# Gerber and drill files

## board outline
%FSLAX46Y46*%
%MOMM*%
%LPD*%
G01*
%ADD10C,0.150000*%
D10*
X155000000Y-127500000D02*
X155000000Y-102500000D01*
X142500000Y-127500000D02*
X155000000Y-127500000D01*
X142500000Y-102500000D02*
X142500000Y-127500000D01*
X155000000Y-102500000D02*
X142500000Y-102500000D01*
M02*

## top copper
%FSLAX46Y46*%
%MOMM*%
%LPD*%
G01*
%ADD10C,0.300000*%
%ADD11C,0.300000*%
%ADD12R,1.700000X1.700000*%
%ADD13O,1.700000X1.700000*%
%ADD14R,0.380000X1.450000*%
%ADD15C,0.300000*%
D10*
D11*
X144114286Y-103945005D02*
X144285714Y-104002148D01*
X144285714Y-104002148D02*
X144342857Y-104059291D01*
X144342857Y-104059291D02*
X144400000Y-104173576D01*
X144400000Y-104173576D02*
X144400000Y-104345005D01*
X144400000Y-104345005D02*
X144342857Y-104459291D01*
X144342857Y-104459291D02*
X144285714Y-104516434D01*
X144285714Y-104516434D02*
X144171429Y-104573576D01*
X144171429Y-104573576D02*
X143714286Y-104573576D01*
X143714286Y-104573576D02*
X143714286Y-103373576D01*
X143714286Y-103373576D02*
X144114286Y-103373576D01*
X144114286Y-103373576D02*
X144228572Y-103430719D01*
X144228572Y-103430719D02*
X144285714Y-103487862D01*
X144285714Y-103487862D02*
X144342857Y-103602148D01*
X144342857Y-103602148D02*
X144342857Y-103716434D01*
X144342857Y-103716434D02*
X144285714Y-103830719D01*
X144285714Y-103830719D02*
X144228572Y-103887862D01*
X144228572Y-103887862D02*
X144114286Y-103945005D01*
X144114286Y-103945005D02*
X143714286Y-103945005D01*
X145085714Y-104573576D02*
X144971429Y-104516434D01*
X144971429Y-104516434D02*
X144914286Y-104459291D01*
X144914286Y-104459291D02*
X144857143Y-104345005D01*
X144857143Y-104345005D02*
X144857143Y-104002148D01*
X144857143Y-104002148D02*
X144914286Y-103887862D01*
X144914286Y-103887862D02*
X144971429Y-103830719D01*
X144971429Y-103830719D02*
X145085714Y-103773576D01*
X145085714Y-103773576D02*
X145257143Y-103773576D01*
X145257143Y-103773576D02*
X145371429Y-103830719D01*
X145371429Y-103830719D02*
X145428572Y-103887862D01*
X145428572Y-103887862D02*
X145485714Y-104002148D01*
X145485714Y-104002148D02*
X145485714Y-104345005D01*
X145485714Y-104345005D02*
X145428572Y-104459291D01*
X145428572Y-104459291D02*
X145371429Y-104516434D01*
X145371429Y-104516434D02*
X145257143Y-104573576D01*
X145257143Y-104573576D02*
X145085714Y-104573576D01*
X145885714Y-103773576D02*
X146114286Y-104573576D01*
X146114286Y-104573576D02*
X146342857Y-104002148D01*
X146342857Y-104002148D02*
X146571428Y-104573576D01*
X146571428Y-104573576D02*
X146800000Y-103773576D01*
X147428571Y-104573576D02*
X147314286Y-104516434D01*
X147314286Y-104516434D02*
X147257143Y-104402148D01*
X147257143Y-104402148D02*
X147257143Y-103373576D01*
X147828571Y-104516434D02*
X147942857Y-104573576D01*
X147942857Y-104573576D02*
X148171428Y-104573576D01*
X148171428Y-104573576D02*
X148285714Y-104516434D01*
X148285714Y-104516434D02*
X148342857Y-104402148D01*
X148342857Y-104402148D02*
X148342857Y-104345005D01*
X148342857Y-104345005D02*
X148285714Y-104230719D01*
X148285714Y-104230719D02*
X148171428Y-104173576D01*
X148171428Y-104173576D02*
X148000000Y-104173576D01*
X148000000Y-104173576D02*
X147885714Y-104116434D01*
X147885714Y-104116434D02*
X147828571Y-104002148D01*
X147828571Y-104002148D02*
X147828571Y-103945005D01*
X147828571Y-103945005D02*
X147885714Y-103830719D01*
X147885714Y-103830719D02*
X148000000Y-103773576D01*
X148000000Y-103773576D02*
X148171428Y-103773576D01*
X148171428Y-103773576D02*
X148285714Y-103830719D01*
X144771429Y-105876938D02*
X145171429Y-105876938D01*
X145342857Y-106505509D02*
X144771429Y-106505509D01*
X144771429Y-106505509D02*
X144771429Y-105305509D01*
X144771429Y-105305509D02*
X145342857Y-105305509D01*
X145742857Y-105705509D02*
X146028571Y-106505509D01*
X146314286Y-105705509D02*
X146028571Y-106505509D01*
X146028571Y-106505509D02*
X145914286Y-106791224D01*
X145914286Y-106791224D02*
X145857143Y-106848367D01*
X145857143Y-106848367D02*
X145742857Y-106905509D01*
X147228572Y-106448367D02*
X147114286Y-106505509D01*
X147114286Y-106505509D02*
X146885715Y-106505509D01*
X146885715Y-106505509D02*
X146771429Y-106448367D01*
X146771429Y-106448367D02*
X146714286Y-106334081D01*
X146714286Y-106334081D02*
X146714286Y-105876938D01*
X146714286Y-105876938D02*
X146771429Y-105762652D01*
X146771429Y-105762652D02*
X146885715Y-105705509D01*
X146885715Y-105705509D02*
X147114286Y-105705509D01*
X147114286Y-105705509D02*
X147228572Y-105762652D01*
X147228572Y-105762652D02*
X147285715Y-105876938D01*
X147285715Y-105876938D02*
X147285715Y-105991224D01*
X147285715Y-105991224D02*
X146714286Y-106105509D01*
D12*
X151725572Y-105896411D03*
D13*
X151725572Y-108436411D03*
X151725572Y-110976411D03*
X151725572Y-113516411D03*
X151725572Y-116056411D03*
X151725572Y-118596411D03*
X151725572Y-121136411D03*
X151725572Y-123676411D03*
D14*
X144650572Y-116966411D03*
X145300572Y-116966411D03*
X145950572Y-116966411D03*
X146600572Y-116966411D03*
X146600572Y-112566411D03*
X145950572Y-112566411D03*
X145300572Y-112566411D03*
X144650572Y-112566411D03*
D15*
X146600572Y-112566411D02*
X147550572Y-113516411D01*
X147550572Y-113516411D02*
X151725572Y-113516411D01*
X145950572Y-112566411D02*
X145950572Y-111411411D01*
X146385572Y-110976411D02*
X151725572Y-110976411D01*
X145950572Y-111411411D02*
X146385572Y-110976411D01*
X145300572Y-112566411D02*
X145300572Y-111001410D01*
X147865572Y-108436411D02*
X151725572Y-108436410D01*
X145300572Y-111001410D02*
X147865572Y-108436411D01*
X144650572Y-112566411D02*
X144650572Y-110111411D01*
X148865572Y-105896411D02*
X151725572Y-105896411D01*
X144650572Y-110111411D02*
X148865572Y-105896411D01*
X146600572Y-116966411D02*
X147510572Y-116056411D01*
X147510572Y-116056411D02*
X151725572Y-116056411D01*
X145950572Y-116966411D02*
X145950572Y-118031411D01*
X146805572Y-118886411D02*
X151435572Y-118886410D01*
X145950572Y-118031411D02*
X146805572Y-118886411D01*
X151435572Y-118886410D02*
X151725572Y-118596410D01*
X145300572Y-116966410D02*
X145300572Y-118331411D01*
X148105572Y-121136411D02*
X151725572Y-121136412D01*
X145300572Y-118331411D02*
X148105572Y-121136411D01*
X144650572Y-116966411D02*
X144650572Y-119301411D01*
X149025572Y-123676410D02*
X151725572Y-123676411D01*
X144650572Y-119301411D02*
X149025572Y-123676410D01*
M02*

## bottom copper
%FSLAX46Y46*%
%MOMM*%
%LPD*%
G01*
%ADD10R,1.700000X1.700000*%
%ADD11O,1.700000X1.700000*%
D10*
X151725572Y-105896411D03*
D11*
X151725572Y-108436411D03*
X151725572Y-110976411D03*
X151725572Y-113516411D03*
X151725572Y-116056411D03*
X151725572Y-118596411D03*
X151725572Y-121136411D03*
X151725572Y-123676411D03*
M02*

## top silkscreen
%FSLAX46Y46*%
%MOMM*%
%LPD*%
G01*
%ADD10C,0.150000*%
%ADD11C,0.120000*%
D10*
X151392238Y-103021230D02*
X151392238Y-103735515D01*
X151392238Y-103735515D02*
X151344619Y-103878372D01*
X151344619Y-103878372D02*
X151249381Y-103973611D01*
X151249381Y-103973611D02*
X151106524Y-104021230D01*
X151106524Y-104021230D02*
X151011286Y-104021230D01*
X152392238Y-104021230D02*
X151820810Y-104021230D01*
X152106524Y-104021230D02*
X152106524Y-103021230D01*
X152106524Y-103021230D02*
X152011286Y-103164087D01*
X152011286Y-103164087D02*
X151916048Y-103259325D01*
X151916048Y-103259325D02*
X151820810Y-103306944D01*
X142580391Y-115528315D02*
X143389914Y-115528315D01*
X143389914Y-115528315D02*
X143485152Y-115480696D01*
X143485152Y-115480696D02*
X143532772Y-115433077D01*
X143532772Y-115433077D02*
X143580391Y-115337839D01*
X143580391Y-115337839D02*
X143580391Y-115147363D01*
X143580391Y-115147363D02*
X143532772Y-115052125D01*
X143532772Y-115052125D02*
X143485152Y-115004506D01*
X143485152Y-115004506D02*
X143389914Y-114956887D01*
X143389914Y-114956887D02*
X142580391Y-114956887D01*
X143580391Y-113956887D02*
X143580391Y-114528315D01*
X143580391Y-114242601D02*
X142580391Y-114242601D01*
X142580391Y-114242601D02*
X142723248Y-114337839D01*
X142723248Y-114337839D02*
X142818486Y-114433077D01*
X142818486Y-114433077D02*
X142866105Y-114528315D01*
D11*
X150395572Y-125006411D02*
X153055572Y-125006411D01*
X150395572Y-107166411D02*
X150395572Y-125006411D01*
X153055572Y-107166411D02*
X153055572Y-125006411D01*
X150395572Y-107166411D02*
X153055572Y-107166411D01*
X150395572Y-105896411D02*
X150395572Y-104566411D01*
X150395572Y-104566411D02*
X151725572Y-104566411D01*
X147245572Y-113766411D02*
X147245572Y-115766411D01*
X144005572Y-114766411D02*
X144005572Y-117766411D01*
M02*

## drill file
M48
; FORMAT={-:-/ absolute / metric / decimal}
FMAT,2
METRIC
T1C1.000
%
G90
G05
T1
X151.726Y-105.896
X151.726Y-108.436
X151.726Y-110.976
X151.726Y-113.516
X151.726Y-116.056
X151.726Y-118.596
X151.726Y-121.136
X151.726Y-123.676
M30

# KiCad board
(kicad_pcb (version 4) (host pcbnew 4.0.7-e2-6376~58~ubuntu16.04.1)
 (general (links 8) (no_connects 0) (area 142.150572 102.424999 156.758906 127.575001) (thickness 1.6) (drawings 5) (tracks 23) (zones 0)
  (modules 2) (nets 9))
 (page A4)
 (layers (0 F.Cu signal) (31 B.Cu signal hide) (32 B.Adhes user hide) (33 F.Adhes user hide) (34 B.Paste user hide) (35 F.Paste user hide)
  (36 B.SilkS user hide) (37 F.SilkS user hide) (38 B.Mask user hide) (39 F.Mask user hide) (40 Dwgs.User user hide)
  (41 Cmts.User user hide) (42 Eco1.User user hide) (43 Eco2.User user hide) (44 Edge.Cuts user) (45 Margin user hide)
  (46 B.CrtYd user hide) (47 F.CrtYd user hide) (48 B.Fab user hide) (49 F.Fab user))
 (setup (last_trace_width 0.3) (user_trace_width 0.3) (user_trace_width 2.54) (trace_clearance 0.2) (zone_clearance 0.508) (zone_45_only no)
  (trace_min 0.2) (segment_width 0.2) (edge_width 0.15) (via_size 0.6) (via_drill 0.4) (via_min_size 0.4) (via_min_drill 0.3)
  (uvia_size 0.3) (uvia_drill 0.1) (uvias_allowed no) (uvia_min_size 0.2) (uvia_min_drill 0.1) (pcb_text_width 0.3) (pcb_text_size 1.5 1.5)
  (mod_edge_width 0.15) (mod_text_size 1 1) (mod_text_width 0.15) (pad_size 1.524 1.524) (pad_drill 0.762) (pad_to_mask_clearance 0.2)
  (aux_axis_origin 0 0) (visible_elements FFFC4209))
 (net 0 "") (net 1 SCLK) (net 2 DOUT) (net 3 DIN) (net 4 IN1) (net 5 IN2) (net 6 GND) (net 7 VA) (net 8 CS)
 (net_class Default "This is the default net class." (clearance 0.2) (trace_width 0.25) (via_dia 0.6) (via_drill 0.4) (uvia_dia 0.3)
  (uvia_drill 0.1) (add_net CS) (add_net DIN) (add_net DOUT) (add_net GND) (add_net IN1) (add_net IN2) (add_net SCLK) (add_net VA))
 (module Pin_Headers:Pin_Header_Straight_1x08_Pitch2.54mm (layer F.Cu) (at 151.725572 105.896411)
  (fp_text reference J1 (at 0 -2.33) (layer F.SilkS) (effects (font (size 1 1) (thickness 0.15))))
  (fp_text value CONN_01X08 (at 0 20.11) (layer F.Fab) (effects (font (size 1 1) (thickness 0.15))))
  (fp_line (start -1.33 19.11) (end 1.33 19.11) (layer F.SilkS) (width 0.12))
  (fp_line (start -1.33 1.27) (end -1.33 19.11) (layer F.SilkS) (width 0.12))
  (fp_line (start 1.33 1.27) (end 1.33 19.11) (layer F.SilkS) (width 0.12))
  (fp_line (start -1.33 1.27) (end 1.33 1.27) (layer F.SilkS) (width 0.12))
  (fp_line (start -1.33 0) (end -1.33 -1.33) (layer F.SilkS) (width 0.12))
  (fp_line (start -1.33 -1.33) (end 0 -1.33) (layer F.SilkS) (width 0.12))
  (pad 1 thru_hole rect (at 0 0) (size 1.7 1.7) (drill 1) (layers *.Cu *.Mask) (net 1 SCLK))
  (pad 2 thru_hole oval (at 0 2.54) (size 1.7 1.7) (drill 1) (layers *.Cu *.Mask) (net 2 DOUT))
  (pad 3 thru_hole oval (at 0 5.08) (size 1.7 1.7) (drill 1) (layers *.Cu *.Mask) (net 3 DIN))
  (pad 4 thru_hole oval (at 0 7.62) (size 1.7 1.7) (drill 1) (layers *.Cu *.Mask) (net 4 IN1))
  (pad 5 thru_hole oval (at 0 10.16) (size 1.7 1.7) (drill 1) (layers *.Cu *.Mask) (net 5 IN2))
  (pad 6 thru_hole oval (at 0 12.7) (size 1.7 1.7) (drill 1) (layers *.Cu *.Mask) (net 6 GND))
  (pad 7 thru_hole oval (at 0 15.24) (size 1.7 1.7) (drill 1) (layers *.Cu *.Mask) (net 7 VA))
  (pad 8 thru_hole oval (at 0 17.78) (size 1.7 1.7) (drill 1) (layers *.Cu *.Mask) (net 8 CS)))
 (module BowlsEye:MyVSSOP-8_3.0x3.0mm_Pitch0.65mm (layer F.Cu) (at 145.625572 114.766411 90)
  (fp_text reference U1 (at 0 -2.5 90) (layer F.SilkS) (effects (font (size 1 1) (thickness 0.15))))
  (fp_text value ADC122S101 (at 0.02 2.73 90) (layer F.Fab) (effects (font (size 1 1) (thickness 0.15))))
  (fp_line (start 1 1.62) (end -1 1.62) (layer F.SilkS) (width 0.12))
  (fp_line (start 0 -1.62) (end -3 -1.62) (layer F.SilkS) (width 0.12))
  (pad 1 smd rect (at -2.2 -0.975) (size 0.38 1.45) (layers F.Cu F.Paste F.Mask) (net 8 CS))
  (pad 2 smd rect (at -2.2 -0.325) (size 0.38 1.45) (layers F.Cu F.Paste F.Mask) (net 7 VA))
  (pad 3 smd rect (at -2.2 0.325) (size 0.38 1.45) (layers F.Cu F.Paste F.Mask) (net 6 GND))
  (pad 4 smd rect (at -2.2 0.975) (size 0.38 1.45) (layers F.Cu F.Paste F.Mask) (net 5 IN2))
  (pad 5 smd rect (at 2.2 0.975) (size 0.38 1.45) (layers F.Cu F.Paste F.Mask) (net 4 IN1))
  (pad 6 smd rect (at 2.2 0.325) (size 0.38 1.45) (layers F.Cu F.Paste F.Mask) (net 3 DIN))
  (pad 7 smd rect (at 2.2 -0.325) (size 0.38 1.45) (layers F.Cu F.Paste F.Mask) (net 2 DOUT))
  (pad 8 smd rect (at 2.2 -0.975) (size 0.38 1.45) (layers F.Cu F.Paste F.Mask) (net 1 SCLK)))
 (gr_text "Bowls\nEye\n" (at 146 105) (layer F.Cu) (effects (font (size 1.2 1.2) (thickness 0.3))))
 (gr_line (start 155 127.5) (end 155 102.5) (angle 90) (layer Edge.Cuts) (width 0.15))
 (gr_line (start 142.5 127.5) (end 155 127.5) (angle 90) (layer Edge.Cuts) (width 0.15))
 (gr_line (start 142.5 102.5) (end 142.5 127.5) (angle 90) (layer Edge.Cuts) (width 0.15))
 (gr_line (start 155 102.5) (end 142.5 102.5) (angle 90) (layer Edge.Cuts) (width 0.15))
 (segment (start 146.600572 112.566411) (end 147.550572 113.516411) (width 0.3) (layer F.Cu) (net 4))
 (segment (start 147.550572 113.516411) (end 151.725572 113.516411) (width 0.3) (layer F.Cu) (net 4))
 (segment (start 145.950572 112.566411) (end 145.950572 111.411411) (width 0.3) (layer F.Cu) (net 3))
 (segment (start 146.385572 110.976411) (end 151.725572 110.976411) (width 0.3) (layer F.Cu) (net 3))
 (segment (start 145.950572 111.411411) (end 146.385572 110.976411) (width 0.3) (layer F.Cu) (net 3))
 (segment (start 145.300572 112.566411) (end 145.300572 111.00141) (width 0.3) (layer F.Cu) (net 2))
 (segment (start 147.865572 108.436411) (end 151.725572 108.43641) (width 0.3) (layer F.Cu) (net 2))
 (segment (start 145.300572 111.00141) (end 147.865572 108.436411) (width 0.3) (layer F.Cu) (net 2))
 (segment (start 144.650572 112.566411) (end 144.650572 110.111411) (width 0.3) (layer F.Cu) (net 1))
 (segment (start 148.865572 105.896411) (end 151.725572 105.896411) (width 0.3) (layer F.Cu) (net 1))
 (segment (start 144.650572 110.111411) (end 148.865572 105.896411) (width 0.3) (layer F.Cu) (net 1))
 (segment (start 146.600572 116.966411) (end 147.510572 116.056411) (width 0.3) (layer F.Cu) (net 5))
 (segment (start 147.510572 116.056411) (end 151.725572 116.056411) (width 0.3) (layer F.Cu) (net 5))
 (segment (start 145.950572 116.966411) (end 145.950572 118.031411) (width 0.3) (layer F.Cu) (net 6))
 (segment (start 146.805572 118.886411) (end 151.435572 118.88641) (width 0.3) (layer F.Cu) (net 6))
 (segment (start 145.950572 118.031411) (end 146.805572 118.886411) (width 0.3) (layer F.Cu) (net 6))
 (segment (start 151.435572 118.88641) (end 151.725572 118.59641) (width 0.3) (layer F.Cu) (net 6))
 (segment (start 145.300572 116.96641) (end 145.300572 118.331411) (width 0.3) (layer F.Cu) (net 7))
 (segment (start 148.105572 121.136411) (end 151.725572 121.136412) (width 0.3) (layer F.Cu) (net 7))
 (segment (start 145.300572 118.331411) (end 148.105572 121.136411) (width 0.3) (layer F.Cu) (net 7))
 (segment (start 144.650572 116.966411) (end 144.650572 119.301411) (width 0.3) (layer F.Cu) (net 8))
 (segment (start 149.025572 123.67641) (end 151.725572 123.676411) (width 0.3) (layer F.Cu) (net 8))
 (segment (start 144.650572 119.301411) (end 149.025572 123.67641) (width 0.3) (layer F.Cu) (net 8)))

